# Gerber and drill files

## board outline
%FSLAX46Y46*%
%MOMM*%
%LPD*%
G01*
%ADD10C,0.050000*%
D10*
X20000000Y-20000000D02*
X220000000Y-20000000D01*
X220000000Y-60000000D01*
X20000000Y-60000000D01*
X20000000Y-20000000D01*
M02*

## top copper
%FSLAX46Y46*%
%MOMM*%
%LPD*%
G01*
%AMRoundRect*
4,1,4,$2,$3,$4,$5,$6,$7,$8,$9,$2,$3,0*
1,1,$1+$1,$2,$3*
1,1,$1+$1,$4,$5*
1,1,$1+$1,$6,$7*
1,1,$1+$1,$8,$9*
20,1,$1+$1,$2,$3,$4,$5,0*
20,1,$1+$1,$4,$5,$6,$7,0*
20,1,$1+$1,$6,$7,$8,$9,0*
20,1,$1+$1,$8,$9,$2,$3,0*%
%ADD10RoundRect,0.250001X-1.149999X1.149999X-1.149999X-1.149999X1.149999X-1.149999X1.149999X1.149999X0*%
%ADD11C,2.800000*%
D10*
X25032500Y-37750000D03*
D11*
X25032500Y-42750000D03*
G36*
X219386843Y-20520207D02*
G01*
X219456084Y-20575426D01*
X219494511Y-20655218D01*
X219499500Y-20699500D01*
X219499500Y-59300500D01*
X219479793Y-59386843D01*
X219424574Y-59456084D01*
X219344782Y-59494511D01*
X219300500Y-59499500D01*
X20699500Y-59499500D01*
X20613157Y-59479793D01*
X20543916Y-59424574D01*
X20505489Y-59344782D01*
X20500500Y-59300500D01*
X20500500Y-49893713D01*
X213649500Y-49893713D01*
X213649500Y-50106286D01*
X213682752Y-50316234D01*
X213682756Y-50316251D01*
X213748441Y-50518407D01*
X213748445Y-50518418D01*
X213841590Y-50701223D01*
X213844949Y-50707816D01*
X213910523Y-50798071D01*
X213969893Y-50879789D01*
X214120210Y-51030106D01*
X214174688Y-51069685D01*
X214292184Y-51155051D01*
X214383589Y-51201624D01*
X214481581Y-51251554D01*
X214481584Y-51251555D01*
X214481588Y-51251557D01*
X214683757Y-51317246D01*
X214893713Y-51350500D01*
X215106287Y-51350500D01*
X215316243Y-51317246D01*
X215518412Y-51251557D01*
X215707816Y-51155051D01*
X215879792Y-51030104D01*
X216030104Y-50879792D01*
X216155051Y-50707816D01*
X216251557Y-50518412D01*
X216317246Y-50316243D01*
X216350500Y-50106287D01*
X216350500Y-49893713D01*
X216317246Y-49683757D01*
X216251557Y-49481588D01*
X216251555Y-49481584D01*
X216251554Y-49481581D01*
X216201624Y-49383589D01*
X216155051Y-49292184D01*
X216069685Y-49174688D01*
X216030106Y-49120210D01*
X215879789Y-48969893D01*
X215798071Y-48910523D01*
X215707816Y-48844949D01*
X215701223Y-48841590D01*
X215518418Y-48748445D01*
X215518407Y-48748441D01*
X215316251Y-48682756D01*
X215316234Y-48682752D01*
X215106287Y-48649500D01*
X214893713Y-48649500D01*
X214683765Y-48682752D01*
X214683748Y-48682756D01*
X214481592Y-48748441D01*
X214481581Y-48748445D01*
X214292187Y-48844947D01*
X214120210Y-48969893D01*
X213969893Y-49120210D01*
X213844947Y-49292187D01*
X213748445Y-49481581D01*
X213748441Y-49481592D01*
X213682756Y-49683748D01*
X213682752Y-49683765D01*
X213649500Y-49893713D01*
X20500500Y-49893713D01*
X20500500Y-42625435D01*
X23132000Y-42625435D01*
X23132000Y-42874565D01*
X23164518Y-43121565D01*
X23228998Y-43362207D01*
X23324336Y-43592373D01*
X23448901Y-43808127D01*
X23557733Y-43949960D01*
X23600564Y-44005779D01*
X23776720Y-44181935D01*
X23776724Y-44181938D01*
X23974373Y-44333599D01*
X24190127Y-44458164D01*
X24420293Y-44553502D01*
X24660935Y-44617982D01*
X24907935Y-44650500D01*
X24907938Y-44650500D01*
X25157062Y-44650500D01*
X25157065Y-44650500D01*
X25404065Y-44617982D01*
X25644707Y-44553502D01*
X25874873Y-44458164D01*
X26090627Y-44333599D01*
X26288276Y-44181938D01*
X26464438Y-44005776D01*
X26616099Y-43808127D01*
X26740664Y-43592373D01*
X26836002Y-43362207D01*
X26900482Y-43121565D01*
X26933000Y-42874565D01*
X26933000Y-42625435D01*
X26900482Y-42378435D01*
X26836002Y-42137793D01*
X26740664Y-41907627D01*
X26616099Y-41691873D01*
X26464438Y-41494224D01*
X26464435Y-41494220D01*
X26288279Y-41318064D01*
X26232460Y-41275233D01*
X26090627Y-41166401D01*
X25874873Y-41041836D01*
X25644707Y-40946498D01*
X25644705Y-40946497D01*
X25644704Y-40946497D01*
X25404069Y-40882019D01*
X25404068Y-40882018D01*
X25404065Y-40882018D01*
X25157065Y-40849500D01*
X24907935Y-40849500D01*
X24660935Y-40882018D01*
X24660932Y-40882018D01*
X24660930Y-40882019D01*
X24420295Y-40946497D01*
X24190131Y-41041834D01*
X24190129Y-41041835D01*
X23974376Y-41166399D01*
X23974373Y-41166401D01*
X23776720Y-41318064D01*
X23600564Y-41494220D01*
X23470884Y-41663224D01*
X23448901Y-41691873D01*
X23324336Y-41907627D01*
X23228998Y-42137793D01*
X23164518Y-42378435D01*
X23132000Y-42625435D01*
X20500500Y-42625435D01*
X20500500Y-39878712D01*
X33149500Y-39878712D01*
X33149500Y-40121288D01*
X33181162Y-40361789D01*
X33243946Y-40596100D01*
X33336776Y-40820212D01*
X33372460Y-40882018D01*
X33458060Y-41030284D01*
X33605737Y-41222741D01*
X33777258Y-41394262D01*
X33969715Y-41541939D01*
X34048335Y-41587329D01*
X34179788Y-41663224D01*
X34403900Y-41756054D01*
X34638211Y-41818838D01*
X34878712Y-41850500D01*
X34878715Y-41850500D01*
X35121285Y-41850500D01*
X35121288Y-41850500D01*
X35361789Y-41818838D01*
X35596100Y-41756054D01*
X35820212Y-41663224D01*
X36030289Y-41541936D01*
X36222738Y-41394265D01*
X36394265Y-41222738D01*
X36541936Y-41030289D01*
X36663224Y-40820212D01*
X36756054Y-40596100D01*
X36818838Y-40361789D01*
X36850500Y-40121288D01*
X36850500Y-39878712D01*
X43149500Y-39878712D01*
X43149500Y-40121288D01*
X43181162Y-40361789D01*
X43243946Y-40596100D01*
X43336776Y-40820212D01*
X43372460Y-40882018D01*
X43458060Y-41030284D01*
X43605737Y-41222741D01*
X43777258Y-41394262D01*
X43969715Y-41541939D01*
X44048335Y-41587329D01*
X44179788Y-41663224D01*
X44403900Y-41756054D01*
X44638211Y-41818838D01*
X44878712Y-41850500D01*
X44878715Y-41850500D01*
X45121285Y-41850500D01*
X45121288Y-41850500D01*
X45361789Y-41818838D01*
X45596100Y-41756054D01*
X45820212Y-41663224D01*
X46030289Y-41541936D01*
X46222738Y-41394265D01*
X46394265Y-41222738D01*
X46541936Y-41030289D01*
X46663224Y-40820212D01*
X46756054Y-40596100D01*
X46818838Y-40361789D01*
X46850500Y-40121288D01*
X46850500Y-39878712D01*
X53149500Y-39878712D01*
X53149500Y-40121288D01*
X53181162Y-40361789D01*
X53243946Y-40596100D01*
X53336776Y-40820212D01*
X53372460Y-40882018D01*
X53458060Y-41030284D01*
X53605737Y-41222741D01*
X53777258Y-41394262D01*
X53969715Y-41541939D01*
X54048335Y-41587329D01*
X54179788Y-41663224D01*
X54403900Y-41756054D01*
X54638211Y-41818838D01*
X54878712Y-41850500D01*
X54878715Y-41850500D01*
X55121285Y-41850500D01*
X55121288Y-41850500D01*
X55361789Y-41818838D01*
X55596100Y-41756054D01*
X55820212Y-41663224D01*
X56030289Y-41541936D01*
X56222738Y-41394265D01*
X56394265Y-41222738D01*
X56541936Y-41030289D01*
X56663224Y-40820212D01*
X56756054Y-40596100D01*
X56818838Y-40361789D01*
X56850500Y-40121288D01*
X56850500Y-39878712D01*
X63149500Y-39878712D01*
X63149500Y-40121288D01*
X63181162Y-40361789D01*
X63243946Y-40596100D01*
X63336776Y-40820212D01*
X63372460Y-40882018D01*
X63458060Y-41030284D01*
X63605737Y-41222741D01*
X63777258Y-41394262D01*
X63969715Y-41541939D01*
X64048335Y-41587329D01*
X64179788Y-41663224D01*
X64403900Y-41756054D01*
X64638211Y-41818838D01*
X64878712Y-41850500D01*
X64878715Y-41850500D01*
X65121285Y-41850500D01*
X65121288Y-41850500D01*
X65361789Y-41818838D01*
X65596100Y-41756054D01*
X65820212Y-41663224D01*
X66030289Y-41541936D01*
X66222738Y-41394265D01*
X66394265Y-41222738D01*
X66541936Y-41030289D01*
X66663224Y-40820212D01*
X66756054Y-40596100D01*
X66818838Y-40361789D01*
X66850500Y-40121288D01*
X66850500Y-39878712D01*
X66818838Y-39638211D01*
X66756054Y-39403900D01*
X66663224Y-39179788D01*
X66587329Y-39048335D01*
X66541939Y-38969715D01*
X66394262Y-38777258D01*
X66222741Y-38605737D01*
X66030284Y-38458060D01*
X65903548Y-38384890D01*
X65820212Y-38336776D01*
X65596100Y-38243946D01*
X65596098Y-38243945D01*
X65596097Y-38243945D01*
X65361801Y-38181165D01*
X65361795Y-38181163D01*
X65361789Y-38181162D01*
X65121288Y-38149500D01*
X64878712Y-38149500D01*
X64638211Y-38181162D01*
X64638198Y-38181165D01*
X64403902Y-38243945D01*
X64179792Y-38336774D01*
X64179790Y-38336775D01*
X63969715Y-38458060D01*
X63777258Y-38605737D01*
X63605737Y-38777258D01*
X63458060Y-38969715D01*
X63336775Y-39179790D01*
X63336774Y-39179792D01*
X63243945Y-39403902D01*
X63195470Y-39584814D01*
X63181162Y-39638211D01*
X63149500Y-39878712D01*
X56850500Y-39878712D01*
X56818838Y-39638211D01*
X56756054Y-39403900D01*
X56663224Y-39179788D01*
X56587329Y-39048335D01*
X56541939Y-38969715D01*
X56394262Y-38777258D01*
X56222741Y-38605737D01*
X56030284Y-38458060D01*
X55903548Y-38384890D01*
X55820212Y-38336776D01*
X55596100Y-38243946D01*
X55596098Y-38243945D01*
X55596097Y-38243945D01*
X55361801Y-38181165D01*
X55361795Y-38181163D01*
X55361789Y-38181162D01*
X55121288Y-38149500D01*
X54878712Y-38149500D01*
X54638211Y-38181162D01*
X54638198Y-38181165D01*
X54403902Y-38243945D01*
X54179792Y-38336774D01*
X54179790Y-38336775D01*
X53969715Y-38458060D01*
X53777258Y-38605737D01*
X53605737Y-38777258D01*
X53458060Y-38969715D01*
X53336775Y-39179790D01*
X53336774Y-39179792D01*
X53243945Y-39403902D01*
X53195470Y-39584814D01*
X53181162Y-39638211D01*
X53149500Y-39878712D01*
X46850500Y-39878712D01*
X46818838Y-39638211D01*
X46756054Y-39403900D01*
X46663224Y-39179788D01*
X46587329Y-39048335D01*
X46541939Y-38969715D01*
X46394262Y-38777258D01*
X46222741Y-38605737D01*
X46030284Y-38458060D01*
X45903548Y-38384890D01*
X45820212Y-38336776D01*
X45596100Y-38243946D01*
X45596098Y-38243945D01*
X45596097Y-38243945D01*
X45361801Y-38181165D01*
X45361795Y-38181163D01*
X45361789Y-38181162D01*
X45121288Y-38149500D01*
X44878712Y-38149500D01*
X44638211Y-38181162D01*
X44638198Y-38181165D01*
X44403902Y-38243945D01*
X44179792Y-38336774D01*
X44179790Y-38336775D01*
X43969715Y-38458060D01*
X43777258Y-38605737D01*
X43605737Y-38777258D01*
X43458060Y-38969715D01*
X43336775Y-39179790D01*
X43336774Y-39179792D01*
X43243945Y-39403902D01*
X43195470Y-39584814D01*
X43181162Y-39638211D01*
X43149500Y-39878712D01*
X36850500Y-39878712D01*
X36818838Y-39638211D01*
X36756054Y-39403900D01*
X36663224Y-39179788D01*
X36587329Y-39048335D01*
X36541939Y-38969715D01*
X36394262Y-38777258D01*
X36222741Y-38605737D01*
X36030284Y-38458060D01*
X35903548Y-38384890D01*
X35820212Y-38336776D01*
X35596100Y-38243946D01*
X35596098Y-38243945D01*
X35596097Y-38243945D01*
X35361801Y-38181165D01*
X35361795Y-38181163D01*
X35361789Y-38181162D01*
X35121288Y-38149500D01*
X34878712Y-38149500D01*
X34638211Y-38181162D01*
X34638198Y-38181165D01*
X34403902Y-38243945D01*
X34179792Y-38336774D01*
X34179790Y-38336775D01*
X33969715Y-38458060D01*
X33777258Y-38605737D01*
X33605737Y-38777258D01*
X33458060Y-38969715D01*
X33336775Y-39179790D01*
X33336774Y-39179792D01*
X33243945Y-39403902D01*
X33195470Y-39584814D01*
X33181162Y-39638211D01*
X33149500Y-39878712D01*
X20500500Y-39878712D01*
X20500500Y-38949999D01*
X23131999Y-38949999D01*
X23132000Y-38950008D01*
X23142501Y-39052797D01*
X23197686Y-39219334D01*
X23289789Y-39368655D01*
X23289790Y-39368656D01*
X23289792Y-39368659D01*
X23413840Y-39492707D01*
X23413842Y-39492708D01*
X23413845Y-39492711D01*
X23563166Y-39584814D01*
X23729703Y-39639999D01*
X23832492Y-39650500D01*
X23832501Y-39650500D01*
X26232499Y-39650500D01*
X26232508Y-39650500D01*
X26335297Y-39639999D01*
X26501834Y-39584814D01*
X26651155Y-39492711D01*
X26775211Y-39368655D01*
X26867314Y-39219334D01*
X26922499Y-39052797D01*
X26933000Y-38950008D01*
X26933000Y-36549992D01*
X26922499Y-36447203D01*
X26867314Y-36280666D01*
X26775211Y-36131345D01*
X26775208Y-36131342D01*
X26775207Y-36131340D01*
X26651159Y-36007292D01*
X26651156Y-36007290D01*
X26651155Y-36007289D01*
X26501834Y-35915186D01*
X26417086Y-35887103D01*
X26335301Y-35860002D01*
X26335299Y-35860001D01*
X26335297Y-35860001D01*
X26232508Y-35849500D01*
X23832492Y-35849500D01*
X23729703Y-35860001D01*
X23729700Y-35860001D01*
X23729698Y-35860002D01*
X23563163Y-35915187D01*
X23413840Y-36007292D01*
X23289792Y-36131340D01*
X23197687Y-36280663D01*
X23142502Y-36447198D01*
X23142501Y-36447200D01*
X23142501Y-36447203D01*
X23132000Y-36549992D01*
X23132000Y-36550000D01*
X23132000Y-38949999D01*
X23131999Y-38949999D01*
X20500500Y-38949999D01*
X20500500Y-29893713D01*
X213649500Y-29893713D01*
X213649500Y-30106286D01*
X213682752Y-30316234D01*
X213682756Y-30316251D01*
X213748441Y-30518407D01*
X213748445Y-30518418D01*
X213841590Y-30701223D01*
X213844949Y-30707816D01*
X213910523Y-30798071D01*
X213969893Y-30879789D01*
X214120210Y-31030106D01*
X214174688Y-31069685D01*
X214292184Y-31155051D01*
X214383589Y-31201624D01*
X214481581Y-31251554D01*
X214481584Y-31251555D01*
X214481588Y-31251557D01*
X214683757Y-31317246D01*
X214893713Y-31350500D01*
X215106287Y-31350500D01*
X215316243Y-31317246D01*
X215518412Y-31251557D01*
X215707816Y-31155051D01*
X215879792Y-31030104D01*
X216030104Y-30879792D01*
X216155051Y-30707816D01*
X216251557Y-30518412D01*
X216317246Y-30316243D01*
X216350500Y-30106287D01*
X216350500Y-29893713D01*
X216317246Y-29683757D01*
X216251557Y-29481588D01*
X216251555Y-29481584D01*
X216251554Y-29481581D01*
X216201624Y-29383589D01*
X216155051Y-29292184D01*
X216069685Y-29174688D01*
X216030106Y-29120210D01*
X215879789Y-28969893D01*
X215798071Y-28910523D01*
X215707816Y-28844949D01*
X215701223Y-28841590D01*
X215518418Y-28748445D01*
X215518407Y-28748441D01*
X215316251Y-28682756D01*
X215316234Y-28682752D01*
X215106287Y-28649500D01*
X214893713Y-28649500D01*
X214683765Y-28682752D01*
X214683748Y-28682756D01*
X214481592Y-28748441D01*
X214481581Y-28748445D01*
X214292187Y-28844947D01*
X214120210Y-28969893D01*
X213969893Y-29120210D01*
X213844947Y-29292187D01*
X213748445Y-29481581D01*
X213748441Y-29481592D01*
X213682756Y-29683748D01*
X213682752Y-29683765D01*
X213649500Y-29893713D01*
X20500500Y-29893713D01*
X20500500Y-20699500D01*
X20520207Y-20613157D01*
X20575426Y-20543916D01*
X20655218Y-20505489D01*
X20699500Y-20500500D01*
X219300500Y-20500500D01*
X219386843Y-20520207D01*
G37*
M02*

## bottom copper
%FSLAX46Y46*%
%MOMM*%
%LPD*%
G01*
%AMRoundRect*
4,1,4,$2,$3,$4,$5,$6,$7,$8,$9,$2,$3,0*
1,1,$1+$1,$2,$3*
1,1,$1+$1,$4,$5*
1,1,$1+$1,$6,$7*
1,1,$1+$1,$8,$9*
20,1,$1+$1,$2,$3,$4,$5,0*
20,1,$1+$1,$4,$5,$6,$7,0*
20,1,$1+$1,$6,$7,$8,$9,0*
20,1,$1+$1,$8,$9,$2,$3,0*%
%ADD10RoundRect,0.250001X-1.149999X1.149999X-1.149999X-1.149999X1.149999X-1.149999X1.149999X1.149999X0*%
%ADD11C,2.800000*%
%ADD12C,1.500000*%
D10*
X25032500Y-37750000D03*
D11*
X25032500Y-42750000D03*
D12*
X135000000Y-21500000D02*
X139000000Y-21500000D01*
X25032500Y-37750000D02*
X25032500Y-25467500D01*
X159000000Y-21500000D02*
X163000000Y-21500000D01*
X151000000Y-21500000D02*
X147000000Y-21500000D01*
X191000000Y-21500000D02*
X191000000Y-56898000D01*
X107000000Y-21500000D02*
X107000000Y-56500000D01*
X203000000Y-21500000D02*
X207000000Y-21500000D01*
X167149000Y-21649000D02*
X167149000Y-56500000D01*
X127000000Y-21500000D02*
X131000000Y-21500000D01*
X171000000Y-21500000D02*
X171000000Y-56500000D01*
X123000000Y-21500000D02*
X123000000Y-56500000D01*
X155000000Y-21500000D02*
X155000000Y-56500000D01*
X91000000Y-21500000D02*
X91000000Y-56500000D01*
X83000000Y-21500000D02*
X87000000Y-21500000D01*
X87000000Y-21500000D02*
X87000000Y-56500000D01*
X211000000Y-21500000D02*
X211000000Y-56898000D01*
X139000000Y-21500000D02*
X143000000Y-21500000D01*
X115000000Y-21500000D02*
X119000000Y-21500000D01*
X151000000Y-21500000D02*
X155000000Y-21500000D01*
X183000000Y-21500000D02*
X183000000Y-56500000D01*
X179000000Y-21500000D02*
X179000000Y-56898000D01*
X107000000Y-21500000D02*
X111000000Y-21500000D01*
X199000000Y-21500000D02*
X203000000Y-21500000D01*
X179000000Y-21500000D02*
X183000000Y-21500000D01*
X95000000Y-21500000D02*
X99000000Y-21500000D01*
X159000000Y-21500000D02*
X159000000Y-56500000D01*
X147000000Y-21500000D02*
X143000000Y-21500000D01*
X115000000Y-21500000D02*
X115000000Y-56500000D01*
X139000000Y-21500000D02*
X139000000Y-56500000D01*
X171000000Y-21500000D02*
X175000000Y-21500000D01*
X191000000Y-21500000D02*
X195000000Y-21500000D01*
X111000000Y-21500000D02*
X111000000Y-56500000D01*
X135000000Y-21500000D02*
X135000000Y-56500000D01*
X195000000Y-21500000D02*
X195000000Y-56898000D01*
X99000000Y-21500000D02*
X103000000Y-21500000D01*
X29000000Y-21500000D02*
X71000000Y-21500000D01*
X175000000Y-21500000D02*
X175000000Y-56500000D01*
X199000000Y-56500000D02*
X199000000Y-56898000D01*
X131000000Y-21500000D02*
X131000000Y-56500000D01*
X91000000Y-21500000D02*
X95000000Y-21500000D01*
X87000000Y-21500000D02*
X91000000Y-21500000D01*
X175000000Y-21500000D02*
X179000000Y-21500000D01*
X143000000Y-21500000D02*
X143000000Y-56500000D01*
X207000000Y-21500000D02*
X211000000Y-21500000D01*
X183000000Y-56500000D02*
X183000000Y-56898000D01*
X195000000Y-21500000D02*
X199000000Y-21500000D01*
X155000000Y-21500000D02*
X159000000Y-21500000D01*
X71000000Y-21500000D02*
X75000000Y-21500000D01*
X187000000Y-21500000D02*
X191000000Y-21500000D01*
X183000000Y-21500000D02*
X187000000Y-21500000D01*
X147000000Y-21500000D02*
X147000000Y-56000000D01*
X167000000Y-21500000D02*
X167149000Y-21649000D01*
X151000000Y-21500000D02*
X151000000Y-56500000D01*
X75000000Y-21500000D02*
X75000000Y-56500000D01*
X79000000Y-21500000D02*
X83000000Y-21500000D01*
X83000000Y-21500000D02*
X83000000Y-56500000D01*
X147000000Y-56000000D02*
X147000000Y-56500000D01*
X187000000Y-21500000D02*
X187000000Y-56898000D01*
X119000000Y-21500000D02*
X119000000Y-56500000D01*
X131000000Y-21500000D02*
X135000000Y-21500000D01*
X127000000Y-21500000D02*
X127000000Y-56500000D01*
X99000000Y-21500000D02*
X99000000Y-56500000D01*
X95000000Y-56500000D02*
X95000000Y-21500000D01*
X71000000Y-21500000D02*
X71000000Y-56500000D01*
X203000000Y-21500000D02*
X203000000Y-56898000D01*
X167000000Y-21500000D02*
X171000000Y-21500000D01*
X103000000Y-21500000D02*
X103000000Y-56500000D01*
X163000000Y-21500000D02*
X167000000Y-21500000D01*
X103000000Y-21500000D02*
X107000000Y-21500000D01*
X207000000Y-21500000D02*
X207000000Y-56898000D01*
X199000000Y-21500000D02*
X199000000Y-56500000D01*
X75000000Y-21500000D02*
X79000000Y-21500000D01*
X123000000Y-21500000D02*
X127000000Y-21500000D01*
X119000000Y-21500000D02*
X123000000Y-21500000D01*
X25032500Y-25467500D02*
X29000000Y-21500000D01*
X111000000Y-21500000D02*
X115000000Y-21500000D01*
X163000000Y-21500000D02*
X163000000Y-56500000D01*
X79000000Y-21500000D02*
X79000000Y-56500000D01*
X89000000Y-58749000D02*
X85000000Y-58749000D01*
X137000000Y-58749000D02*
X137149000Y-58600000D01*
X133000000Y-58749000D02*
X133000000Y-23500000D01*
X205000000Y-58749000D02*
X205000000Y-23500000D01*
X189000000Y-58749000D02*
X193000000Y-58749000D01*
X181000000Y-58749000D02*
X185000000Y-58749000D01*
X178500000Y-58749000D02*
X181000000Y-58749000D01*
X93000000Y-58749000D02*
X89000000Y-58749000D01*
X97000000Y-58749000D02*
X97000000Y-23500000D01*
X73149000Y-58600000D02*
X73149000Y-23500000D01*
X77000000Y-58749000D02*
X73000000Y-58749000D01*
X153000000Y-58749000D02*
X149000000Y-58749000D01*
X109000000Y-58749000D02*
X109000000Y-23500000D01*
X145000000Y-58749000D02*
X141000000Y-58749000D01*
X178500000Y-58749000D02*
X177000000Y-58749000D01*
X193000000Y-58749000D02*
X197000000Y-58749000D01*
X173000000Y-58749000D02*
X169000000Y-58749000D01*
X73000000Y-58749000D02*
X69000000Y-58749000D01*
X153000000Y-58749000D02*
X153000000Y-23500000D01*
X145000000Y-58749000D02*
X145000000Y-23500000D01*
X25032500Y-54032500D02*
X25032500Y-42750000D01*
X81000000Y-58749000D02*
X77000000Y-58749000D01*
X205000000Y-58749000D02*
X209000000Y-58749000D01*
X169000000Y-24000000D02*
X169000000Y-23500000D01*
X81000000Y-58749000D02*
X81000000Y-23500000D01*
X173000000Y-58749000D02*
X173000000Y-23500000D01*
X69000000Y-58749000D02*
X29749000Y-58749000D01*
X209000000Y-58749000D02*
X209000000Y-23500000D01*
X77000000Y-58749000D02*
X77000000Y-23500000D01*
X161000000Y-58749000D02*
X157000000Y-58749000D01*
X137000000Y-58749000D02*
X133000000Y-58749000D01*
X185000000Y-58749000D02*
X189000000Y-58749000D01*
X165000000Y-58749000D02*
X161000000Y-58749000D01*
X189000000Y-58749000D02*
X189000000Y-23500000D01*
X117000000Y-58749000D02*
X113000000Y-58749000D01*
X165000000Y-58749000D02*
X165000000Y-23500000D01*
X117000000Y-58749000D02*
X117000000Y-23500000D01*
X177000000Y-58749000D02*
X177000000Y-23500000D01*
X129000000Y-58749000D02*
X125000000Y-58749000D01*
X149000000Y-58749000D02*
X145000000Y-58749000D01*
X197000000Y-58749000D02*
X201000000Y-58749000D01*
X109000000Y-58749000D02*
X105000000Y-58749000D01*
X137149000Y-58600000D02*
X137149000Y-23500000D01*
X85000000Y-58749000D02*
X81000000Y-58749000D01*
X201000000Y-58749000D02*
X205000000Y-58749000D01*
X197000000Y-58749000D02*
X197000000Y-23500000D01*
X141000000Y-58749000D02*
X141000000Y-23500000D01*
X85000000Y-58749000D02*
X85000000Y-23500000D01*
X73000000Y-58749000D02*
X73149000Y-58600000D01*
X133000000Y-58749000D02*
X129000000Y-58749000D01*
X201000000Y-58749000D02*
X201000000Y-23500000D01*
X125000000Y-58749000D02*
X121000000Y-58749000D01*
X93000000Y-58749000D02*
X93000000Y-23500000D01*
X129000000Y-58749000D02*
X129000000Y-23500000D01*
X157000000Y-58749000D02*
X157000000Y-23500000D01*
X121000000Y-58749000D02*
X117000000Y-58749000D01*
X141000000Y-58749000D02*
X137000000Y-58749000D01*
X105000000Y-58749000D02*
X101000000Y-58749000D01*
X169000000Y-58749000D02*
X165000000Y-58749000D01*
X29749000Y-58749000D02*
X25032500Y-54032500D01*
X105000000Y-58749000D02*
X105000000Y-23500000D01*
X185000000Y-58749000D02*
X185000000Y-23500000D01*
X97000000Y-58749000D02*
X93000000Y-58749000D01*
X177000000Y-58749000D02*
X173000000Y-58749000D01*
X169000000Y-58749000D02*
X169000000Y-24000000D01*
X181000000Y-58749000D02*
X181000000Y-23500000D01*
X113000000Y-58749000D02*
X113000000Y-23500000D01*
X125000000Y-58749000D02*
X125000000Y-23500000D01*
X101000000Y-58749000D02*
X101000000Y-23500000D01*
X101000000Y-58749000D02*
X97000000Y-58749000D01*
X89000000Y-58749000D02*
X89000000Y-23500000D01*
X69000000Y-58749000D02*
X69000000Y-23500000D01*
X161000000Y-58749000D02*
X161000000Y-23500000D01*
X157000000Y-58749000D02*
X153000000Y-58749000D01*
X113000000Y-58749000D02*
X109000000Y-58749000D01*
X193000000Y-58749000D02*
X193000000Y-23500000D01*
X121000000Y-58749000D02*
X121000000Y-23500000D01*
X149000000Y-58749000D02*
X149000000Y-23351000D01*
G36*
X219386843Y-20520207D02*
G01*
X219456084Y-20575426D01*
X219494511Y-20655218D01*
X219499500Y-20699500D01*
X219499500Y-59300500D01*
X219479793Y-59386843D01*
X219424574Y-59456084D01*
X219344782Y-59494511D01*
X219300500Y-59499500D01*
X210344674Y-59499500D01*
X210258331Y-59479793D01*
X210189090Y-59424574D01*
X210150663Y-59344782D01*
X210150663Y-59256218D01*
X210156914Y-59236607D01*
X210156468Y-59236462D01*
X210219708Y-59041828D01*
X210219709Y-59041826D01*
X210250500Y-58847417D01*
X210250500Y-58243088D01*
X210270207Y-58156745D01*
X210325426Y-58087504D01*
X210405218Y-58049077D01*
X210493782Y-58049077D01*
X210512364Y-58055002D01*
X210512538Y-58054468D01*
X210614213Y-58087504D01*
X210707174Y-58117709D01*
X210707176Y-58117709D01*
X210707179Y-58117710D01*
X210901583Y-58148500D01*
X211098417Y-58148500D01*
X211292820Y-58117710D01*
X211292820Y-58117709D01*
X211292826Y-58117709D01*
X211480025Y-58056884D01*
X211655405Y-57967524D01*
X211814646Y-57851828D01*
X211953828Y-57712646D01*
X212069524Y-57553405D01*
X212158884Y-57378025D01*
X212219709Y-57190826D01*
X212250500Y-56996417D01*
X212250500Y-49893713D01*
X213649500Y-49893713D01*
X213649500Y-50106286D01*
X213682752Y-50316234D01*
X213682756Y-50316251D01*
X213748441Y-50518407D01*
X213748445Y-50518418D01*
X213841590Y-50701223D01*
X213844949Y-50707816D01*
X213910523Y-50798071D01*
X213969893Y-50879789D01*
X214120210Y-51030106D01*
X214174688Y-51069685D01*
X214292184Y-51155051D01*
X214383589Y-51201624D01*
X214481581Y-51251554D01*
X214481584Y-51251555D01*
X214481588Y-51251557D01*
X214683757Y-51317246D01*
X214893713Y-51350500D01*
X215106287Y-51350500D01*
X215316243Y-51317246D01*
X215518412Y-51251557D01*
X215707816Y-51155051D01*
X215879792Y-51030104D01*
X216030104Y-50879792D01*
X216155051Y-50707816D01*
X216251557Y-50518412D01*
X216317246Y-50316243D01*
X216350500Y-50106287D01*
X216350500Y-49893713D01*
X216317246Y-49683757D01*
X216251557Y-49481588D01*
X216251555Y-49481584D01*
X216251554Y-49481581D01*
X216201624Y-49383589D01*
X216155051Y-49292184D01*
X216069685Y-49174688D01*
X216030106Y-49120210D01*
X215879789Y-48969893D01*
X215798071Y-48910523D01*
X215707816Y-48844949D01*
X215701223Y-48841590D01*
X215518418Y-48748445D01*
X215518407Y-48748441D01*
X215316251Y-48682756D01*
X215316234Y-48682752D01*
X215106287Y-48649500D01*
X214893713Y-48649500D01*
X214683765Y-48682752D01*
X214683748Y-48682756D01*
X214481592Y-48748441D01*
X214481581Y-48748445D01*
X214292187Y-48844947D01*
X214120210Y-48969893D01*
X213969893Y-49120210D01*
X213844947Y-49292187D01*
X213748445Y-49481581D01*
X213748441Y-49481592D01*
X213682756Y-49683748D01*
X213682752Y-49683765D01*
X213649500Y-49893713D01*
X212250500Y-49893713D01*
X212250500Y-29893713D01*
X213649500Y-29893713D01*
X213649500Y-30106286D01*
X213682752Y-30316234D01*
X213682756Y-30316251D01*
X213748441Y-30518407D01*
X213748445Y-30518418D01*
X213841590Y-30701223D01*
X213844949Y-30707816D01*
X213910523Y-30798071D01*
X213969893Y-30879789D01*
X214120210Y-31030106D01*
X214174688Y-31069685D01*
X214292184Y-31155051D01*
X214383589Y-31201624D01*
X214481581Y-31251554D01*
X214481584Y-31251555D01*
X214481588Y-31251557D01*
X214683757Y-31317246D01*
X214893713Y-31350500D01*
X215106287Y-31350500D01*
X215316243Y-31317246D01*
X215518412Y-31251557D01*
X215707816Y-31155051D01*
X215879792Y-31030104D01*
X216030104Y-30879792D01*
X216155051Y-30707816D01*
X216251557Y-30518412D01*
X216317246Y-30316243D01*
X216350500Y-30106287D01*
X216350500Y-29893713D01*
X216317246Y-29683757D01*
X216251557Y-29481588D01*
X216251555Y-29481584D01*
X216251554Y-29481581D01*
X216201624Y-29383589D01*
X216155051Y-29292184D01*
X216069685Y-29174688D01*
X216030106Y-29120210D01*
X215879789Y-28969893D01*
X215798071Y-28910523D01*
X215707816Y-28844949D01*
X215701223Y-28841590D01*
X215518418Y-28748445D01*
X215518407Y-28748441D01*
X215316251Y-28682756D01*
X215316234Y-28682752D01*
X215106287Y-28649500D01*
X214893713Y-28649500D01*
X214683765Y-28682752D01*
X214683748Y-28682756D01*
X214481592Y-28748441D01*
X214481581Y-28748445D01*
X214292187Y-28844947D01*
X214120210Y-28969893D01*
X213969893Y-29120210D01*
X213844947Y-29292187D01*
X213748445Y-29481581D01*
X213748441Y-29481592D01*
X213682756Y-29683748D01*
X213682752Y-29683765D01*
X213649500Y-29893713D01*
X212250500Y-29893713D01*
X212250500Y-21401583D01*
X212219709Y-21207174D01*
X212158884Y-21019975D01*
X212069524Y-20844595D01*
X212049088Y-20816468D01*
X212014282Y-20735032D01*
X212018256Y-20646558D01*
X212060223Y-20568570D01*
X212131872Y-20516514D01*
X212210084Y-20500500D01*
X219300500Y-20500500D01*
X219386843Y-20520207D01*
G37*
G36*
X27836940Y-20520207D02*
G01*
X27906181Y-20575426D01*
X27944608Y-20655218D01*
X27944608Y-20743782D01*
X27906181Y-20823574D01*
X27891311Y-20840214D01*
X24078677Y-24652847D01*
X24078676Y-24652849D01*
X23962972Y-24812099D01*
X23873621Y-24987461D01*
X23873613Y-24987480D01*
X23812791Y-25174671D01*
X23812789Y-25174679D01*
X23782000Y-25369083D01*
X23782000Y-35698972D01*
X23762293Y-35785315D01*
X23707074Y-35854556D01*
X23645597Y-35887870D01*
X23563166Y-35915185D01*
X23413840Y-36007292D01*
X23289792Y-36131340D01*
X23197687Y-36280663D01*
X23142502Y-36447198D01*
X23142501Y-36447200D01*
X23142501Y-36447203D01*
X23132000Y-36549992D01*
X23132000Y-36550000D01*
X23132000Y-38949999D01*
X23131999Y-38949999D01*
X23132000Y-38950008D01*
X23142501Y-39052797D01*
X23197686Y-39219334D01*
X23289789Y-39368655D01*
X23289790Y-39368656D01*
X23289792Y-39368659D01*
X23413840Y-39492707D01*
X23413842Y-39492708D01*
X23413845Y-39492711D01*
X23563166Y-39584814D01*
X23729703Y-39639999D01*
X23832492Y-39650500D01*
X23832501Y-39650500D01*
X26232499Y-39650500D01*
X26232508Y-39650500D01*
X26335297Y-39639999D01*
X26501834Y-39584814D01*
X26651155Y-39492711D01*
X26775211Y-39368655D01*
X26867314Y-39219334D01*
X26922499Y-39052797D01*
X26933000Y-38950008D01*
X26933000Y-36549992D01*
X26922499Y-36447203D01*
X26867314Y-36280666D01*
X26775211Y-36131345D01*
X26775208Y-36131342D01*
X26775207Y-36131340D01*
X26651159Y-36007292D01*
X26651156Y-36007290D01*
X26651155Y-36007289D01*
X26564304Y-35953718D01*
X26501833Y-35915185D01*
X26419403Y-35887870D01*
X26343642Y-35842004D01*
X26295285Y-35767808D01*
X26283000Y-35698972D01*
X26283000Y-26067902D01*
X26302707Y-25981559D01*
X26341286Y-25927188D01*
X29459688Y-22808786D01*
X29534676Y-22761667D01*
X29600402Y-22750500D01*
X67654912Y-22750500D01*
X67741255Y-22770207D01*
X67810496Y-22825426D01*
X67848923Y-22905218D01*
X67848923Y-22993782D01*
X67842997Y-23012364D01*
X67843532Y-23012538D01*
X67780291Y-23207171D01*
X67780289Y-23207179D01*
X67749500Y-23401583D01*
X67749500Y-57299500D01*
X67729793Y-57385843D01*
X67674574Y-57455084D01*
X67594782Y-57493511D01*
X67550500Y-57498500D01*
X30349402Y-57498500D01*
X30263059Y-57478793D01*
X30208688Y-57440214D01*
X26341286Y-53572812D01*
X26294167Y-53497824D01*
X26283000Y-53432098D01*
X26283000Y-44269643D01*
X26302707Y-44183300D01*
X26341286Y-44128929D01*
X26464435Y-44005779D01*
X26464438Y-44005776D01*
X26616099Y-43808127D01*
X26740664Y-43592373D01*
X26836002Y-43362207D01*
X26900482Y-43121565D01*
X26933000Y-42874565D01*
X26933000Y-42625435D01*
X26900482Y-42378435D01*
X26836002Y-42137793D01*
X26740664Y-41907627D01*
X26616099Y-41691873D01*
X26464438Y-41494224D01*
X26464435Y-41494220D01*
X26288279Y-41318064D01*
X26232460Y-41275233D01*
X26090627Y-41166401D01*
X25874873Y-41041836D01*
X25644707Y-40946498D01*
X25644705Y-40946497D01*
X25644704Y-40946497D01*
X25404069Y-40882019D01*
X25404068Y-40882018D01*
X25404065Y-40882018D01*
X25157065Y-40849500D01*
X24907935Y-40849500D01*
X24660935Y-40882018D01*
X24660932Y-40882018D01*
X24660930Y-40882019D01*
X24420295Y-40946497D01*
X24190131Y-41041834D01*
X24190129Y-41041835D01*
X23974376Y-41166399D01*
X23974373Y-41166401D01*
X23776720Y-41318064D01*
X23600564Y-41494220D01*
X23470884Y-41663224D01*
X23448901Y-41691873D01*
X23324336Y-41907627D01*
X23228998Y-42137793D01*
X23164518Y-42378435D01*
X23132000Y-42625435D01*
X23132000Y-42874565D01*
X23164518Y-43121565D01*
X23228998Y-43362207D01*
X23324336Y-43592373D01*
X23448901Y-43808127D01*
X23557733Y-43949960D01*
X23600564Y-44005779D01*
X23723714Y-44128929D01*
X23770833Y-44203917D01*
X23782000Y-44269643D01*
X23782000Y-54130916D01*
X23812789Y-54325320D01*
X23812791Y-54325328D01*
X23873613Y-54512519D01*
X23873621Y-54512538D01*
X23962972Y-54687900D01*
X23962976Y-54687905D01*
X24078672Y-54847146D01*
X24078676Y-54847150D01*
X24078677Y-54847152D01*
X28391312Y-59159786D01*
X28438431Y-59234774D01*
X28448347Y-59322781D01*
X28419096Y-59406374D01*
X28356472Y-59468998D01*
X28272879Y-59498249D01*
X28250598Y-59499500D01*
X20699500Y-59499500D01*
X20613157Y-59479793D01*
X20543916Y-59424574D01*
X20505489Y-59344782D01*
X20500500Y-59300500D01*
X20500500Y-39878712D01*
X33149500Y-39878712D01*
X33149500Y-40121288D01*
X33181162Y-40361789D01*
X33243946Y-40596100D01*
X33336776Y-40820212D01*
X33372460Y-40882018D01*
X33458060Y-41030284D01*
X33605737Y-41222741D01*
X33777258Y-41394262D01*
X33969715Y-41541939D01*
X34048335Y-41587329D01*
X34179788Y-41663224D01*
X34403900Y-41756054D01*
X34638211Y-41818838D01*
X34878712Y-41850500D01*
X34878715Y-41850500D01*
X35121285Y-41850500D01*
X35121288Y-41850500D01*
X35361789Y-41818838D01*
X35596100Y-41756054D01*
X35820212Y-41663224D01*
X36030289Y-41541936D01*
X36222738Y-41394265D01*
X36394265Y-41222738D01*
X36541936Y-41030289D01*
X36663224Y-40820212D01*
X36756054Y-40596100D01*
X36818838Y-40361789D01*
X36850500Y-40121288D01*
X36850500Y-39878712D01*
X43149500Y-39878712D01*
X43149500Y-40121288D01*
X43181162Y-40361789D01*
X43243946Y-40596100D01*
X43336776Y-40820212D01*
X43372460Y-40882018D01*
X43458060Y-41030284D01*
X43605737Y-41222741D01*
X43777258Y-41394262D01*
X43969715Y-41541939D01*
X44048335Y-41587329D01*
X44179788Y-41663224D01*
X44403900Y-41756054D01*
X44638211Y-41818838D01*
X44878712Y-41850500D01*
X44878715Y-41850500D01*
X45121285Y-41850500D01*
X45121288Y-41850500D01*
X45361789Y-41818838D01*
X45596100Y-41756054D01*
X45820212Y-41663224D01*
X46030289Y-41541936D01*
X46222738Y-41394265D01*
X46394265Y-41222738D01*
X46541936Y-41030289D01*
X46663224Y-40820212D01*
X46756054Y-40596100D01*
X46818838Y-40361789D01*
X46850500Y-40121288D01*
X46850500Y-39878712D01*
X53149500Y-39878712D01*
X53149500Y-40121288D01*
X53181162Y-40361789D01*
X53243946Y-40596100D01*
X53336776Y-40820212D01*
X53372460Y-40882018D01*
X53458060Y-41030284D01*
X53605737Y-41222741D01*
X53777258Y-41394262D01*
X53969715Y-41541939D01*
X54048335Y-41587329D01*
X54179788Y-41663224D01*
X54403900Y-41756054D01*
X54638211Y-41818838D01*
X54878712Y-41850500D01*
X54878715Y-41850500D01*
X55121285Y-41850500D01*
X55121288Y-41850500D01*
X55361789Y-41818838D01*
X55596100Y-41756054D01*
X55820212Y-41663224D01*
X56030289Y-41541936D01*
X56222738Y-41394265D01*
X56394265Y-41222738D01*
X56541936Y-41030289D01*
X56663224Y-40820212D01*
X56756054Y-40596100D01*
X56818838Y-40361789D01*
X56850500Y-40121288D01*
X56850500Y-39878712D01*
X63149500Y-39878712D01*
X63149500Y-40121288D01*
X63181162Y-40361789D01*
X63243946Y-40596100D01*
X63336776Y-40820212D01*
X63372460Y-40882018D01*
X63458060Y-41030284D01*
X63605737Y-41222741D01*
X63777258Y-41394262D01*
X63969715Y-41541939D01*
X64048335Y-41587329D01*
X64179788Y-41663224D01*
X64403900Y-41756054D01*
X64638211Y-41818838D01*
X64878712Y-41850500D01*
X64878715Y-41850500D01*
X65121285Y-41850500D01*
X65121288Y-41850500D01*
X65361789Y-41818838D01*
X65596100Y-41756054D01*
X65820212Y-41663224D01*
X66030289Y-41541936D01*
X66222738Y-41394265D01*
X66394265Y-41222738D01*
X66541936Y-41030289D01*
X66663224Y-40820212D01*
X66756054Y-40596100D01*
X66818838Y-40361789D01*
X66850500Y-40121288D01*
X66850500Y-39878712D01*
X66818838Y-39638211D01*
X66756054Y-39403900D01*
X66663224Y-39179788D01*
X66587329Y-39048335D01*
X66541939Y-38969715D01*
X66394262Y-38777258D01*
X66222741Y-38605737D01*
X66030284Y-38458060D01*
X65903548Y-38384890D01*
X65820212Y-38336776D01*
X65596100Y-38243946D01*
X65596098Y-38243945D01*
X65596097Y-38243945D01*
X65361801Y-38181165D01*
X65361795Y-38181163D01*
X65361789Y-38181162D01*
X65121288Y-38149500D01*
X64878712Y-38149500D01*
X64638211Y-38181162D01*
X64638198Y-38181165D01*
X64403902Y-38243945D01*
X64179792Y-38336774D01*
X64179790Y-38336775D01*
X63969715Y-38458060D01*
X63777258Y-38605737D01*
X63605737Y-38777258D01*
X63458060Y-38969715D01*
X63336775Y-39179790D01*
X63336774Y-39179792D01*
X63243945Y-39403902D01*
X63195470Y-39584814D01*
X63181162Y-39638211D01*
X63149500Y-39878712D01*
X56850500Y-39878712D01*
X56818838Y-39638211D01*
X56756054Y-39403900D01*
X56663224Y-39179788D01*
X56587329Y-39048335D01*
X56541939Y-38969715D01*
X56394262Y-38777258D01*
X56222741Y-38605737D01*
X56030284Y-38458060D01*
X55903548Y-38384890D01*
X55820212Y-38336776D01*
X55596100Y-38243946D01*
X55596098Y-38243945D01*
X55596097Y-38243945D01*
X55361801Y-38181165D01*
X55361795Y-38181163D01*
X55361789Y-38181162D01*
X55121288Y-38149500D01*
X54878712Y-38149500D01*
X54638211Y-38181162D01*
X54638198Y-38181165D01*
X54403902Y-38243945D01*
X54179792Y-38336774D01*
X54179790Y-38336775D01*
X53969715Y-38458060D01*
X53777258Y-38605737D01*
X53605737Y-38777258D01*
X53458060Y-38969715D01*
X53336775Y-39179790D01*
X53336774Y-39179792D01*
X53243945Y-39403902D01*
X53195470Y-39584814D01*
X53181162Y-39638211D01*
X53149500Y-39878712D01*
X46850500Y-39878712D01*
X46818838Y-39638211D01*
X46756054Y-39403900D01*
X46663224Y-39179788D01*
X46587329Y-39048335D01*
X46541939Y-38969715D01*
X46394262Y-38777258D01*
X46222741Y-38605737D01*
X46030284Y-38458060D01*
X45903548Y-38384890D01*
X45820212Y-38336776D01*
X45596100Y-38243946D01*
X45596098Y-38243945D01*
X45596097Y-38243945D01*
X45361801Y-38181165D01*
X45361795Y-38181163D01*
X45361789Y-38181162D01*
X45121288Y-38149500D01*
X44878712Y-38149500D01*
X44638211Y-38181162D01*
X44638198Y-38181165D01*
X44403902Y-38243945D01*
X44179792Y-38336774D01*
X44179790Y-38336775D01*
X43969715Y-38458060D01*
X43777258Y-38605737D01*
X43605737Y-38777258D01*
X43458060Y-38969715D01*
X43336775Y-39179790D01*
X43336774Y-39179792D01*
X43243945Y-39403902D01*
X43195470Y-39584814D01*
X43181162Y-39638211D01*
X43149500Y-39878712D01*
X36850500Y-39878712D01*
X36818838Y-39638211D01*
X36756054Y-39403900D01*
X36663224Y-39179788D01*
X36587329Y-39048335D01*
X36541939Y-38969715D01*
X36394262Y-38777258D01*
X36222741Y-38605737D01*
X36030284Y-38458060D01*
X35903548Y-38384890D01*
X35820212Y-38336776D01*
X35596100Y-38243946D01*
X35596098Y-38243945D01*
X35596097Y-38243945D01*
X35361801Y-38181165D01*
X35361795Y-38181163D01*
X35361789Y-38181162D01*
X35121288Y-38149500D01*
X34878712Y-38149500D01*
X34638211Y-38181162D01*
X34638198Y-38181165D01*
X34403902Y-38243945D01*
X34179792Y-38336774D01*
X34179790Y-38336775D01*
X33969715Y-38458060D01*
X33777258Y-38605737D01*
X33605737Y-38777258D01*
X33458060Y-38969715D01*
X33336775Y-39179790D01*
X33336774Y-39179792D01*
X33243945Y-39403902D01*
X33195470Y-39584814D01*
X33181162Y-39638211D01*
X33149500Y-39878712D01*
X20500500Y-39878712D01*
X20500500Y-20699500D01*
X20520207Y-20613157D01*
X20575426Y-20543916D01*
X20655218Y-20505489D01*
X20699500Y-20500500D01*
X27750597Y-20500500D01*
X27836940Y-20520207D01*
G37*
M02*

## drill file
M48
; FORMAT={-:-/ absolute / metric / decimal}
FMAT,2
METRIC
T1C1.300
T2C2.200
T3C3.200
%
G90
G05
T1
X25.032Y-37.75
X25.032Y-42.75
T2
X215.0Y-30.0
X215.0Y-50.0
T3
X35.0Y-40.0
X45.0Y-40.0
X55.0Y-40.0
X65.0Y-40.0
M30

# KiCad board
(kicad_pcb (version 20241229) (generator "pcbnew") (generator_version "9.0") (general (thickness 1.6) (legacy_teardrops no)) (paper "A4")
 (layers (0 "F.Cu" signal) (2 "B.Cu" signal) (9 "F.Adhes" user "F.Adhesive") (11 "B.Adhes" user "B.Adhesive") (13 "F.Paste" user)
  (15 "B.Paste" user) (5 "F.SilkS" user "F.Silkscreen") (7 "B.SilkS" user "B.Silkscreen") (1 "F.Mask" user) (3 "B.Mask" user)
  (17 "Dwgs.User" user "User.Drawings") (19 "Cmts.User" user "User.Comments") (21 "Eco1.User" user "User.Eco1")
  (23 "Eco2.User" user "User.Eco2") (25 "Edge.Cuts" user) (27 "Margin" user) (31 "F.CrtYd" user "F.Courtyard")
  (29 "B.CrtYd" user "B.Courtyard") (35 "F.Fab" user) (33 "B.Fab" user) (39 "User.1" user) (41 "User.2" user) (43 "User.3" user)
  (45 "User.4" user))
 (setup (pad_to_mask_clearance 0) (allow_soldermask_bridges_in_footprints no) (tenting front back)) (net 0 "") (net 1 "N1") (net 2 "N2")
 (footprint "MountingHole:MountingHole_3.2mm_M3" (layer "F.Cu") (at 35 40)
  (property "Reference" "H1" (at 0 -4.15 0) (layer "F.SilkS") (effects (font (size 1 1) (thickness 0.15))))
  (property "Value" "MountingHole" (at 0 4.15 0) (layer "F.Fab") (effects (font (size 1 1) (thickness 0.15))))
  (pad "" np_thru_hole circle (at 0 0) (size 3.2 3.2) (drill 3.2) (layers "*.Cu" "*.Mask")))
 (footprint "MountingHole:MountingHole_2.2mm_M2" (layer "F.Cu") (at 215 30)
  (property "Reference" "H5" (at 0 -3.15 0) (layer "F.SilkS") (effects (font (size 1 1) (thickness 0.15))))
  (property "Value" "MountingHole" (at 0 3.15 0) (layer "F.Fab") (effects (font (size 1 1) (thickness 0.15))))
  (pad "" np_thru_hole circle (at 0 0) (size 2.2 2.2) (drill 2.2) (layers "*.Cu" "*.Mask")))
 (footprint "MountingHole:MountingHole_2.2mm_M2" (layer "F.Cu") (at 215 50)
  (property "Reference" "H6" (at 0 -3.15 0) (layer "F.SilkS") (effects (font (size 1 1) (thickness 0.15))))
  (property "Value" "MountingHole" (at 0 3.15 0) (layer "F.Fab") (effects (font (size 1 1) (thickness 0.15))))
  (pad "" np_thru_hole circle (at 0 0) (size 2.2 2.2) (drill 2.2) (layers "*.Cu" "*.Mask")))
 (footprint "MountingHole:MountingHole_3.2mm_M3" (layer "F.Cu") (at 65 40)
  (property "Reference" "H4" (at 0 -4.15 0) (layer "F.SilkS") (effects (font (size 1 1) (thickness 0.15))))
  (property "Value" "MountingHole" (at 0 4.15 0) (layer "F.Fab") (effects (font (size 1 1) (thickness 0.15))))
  (pad "" np_thru_hole circle (at 0 0) (size 3.2 3.2) (drill 3.2) (layers "*.Cu" "*.Mask")))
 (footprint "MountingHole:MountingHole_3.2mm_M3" (layer "F.Cu") (at 55 40)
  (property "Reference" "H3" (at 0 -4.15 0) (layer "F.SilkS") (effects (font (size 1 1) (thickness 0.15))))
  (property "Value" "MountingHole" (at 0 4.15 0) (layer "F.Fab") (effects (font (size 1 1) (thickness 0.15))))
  (pad "" np_thru_hole circle (at 0 0) (size 3.2 3.2) (drill 3.2) (layers "*.Cu" "*.Mask")))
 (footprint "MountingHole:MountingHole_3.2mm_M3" (layer "F.Cu") (at 45 40)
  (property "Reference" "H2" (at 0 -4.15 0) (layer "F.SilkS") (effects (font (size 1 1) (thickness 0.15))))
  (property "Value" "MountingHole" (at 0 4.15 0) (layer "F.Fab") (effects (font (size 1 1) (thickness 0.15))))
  (pad "" np_thru_hole circle (at 0 0) (size 3.2 3.2) (drill 3.2) (layers "*.Cu" "*.Mask")))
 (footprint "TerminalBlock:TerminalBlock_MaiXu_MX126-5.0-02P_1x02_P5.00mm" (layer "F.Cu") (at 25.0325 37.75 -90)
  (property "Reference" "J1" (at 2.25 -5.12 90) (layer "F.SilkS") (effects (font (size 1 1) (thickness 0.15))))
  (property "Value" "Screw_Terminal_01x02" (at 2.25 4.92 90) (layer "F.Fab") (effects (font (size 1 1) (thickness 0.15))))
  (pad "1" thru_hole roundrect (at 0 0 270) (size 2.8 2.8) (drill 1.3) (layers "*.Cu" "*.Mask") (remove_unused_layers no)
   (roundrect_rratio 0.089286) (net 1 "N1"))
  (pad "2" thru_hole circle (at 5 0 270) (size 2.8 2.8) (drill 1.3) (layers "*.Cu" "*.Mask") (remove_unused_layers no) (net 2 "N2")))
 (gr_rect (start 20 20) (end 220 60) (stroke (width 0.05) (type solid)) (fill no) (layer "Edge.Cuts"))
 (segment (start 135 21.5) (end 139 21.5) (width 1.5) (layer "B.Cu") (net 1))
 (segment (start 25.0325 37.75) (end 25.0325 25.4675) (width 1.5) (layer "B.Cu") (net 1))
 (segment (start 159 21.5) (end 163 21.5) (width 1.5) (layer "B.Cu") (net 1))
 (segment (start 151 21.5) (end 147 21.5) (width 1.5) (layer "B.Cu") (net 1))
 (segment (start 191 21.5) (end 191 56.898) (width 1.5) (layer "B.Cu") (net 1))
 (segment (start 107 21.5) (end 107 56.5) (width 1.5) (layer "B.Cu") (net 1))
 (segment (start 203 21.5) (end 207 21.5) (width 1.5) (layer "B.Cu") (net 1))
 (segment (start 167.149 21.649) (end 167.149 56.5) (width 1.5) (layer "B.Cu") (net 1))
 (segment (start 127 21.5) (end 131 21.5) (width 1.5) (layer "B.Cu") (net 1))
 (segment (start 171 21.5) (end 171 56.5) (width 1.5) (layer "B.Cu") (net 1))
 (segment (start 123 21.5) (end 123 56.5) (width 1.5) (layer "B.Cu") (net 1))
 (segment (start 155 21.5) (end 155 56.5) (width 1.5) (layer "B.Cu") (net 1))
 (segment (start 91 21.5) (end 91 56.5) (width 1.5) (layer "B.Cu") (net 1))
 (segment (start 83 21.5) (end 87 21.5) (width 1.5) (layer "B.Cu") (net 1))
 (segment (start 87 21.5) (end 87 56.5) (width 1.5) (layer "B.Cu") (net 1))
 (segment (start 211 21.5) (end 211 56.898) (width 1.5) (layer "B.Cu") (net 1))
 (segment (start 139 21.5) (end 143 21.5) (width 1.5) (layer "B.Cu") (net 1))
 (segment (start 115 21.5) (end 119 21.5) (width 1.5) (layer "B.Cu") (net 1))
 (segment (start 151 21.5) (end 155 21.5) (width 1.5) (layer "B.Cu") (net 1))
 (segment (start 183 21.5) (end 183 56.5) (width 1.5) (layer "B.Cu") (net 1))
 (segment (start 179 21.5) (end 179 56.898) (width 1.5) (layer "B.Cu") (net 1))
 (segment (start 107 21.5) (end 111 21.5) (width 1.5) (layer "B.Cu") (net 1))
 (segment (start 199 21.5) (end 203 21.5) (width 1.5) (layer "B.Cu") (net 1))
 (segment (start 179 21.5) (end 183 21.5) (width 1.5) (layer "B.Cu") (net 1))
 (segment (start 95 21.5) (end 99 21.5) (width 1.5) (layer "B.Cu") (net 1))
 (segment (start 159 21.5) (end 159 56.5) (width 1.5) (layer "B.Cu") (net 1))
 (segment (start 147 21.5) (end 143 21.5) (width 1.5) (layer "B.Cu") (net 1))
 (segment (start 115 21.5) (end 115 56.5) (width 1.5) (layer "B.Cu") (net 1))
 (segment (start 139 21.5) (end 139 56.5) (width 1.5) (layer "B.Cu") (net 1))
 (segment (start 171 21.5) (end 175 21.5) (width 1.5) (layer "B.Cu") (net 1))
 (segment (start 191 21.5) (end 195 21.5) (width 1.5) (layer "B.Cu") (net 1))
 (segment (start 111 21.5) (end 111 56.5) (width 1.5) (layer "B.Cu") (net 1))
 (segment (start 135 21.5) (end 135 56.5) (width 1.5) (layer "B.Cu") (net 1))
 (segment (start 195 21.5) (end 195 56.898) (width 1.5) (layer "B.Cu") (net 1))
 (segment (start 99 21.5) (end 103 21.5) (width 1.5) (layer "B.Cu") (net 1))
 (segment (start 29 21.5) (end 71 21.5) (width 1.5) (layer "B.Cu") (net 1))
 (segment (start 175 21.5) (end 175 56.5) (width 1.5) (layer "B.Cu") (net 1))
 (segment (start 199 56.5) (end 199 56.898) (width 1.5) (layer "B.Cu") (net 1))
 (segment (start 131 21.5) (end 131 56.5) (width 1.5) (layer "B.Cu") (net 1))
 (segment (start 91 21.5) (end 95 21.5) (width 1.5) (layer "B.Cu") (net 1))
 (segment (start 87 21.5) (end 91 21.5) (width 1.5) (layer "B.Cu") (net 1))
 (segment (start 175 21.5) (end 179 21.5) (width 1.5) (layer "B.Cu") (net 1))
 (segment (start 143 21.5) (end 143 56.5) (width 1.5) (layer "B.Cu") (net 1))
 (segment (start 207 21.5) (end 211 21.5) (width 1.5) (layer "B.Cu") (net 1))
 (segment (start 183 56.5) (end 183 56.898) (width 1.5) (layer "B.Cu") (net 1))
 (segment (start 195 21.5) (end 199 21.5) (width 1.5) (layer "B.Cu") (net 1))
 (segment (start 155 21.5) (end 159 21.5) (width 1.5) (layer "B.Cu") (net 1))
 (segment (start 71 21.5) (end 75 21.5) (width 1.5) (layer "B.Cu") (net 1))
 (segment (start 187 21.5) (end 191 21.5) (width 1.5) (layer "B.Cu") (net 1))
 (segment (start 183 21.5) (end 187 21.5) (width 1.5) (layer "B.Cu") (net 1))
 (segment (start 147 21.5) (end 147 56) (width 1.5) (layer "B.Cu") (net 1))
 (segment (start 167 21.5) (end 167.149 21.649) (width 1.5) (layer "B.Cu") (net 1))
 (segment (start 151 21.5) (end 151 56.5) (width 1.5) (layer "B.Cu") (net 1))
 (segment (start 75 21.5) (end 75 56.5) (width 1.5) (layer "B.Cu") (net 1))
 (segment (start 79 21.5) (end 83 21.5) (width 1.5) (layer "B.Cu") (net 1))
 (segment (start 83 21.5) (end 83 56.5) (width 1.5) (layer "B.Cu") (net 1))
 (segment (start 147 56) (end 147 56.5) (width 1.5) (layer "B.Cu") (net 1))
 (segment (start 187 21.5) (end 187 56.898) (width 1.5) (layer "B.Cu") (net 1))
 (segment (start 119 21.5) (end 119 56.5) (width 1.5) (layer "B.Cu") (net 1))
 (segment (start 131 21.5) (end 135 21.5) (width 1.5) (layer "B.Cu") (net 1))
 (segment (start 127 21.5) (end 127 56.5) (width 1.5) (layer "B.Cu") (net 1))
 (segment (start 99 21.5) (end 99 56.5) (width 1.5) (layer "B.Cu") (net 1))
 (segment (start 95 56.5) (end 95 21.5) (width 1.5) (layer "B.Cu") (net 1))
 (segment (start 71 21.5) (end 71 56.5) (width 1.5) (layer "B.Cu") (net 1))
 (segment (start 203 21.5) (end 203 56.898) (width 1.5) (layer "B.Cu") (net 1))
 (segment (start 167 21.5) (end 171 21.5) (width 1.5) (layer "B.Cu") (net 1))
 (segment (start 103 21.5) (end 103 56.5) (width 1.5) (layer "B.Cu") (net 1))
 (segment (start 163 21.5) (end 167 21.5) (width 1.5) (layer "B.Cu") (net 1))
 (segment (start 103 21.5) (end 107 21.5) (width 1.5) (layer "B.Cu") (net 1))
 (segment (start 207 21.5) (end 207 56.898) (width 1.5) (layer "B.Cu") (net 1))
 (segment (start 199 21.5) (end 199 56.5) (width 1.5) (layer "B.Cu") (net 1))
 (segment (start 75 21.5) (end 79 21.5) (width 1.5) (layer "B.Cu") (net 1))
 (segment (start 123 21.5) (end 127 21.5) (width 1.5) (layer "B.Cu") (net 1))
 (segment (start 119 21.5) (end 123 21.5) (width 1.5) (layer "B.Cu") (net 1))
 (segment (start 25.0325 25.4675) (end 29 21.5) (width 1.5) (layer "B.Cu") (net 1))
 (segment (start 111 21.5) (end 115 21.5) (width 1.5) (layer "B.Cu") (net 1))
 (segment (start 163 21.5) (end 163 56.5) (width 1.5) (layer "B.Cu") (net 1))
 (segment (start 79 21.5) (end 79 56.5) (width 1.5) (layer "B.Cu") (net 1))
 (segment (start 89 58.749) (end 85 58.749) (width 1.5) (layer "B.Cu") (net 2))
 (segment (start 137 58.749) (end 137.149 58.6) (width 1.5) (layer "B.Cu") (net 2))
 (segment (start 133 58.749) (end 133 23.5) (width 1.5) (layer "B.Cu") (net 2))
 (segment (start 205 58.749) (end 205 23.5) (width 1.5) (layer "B.Cu") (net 2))
 (segment (start 189 58.749) (end 193 58.749) (width 1.5) (layer "B.Cu") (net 2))
 (segment (start 181 58.749) (end 185 58.749) (width 1.5) (layer "B.Cu") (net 2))
 (segment (start 178.5 58.749) (end 181 58.749) (width 1.5) (layer "B.Cu") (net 2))
 (segment (start 93 58.749) (end 89 58.749) (width 1.5) (layer "B.Cu") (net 2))
 (segment (start 97 58.749) (end 97 23.5) (width 1.5) (layer "B.Cu") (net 2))
 (segment (start 73.149 58.6) (end 73.149 23.5) (width 1.5) (layer "B.Cu") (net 2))
 (segment (start 77 58.749) (end 73 58.749) (width 1.5) (layer "B.Cu") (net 2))
 (segment (start 153 58.749) (end 149 58.749) (width 1.5) (layer "B.Cu") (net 2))
 (segment (start 109 58.749) (end 109 23.5) (width 1.5) (layer "B.Cu") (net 2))
 (segment (start 145 58.749) (end 141 58.749) (width 1.5) (layer "B.Cu") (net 2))
 (segment (start 178.5 58.749) (end 177 58.749) (width 1.5) (layer "B.Cu") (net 2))
 (segment (start 193 58.749) (end 197 58.749) (width 1.5) (layer "B.Cu") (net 2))
 (segment (start 173 58.749) (end 169 58.749) (width 1.5) (layer "B.Cu") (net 2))
 (segment (start 73 58.749) (end 69 58.749) (width 1.5) (layer "B.Cu") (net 2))
 (segment (start 153 58.749) (end 153 23.5) (width 1.5) (layer "B.Cu") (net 2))
 (segment (start 145 58.749) (end 145 23.5) (width 1.5) (layer "B.Cu") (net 2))
 (segment (start 25.0325 54.0325) (end 25.0325 42.75) (width 1.5) (layer "B.Cu") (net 2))
 (segment (start 81 58.749) (end 77 58.749) (width 1.5) (layer "B.Cu") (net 2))
 (segment (start 205 58.749) (end 209 58.749) (width 1.5) (layer "B.Cu") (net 2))
 (segment (start 169 24) (end 169 23.5) (width 1.5) (layer "B.Cu") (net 2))
 (segment (start 81 58.749) (end 81 23.5) (width 1.5) (layer "B.Cu") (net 2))
 (segment (start 173 58.749) (end 173 23.5) (width 1.5) (layer "B.Cu") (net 2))
 (segment (start 69 58.749) (end 29.749 58.749) (width 1.5) (layer "B.Cu") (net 2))
 (segment (start 209 58.749) (end 209 23.5) (width 1.5) (layer "B.Cu") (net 2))
 (segment (start 77 58.749) (end 77 23.5) (width 1.5) (layer "B.Cu") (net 2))
 (segment (start 161 58.749) (end 157 58.749) (width 1.5) (layer "B.Cu") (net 2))
 (segment (start 137 58.749) (end 133 58.749) (width 1.5) (layer "B.Cu") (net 2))
 (segment (start 185 58.749) (end 189 58.749) (width 1.5) (layer "B.Cu") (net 2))
 (segment (start 165 58.749) (end 161 58.749) (width 1.5) (layer "B.Cu") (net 2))
 (segment (start 189 58.749) (end 189 23.5) (width 1.5) (layer "B.Cu") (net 2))
 (segment (start 117 58.749) (end 113 58.749) (width 1.5) (layer "B.Cu") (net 2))
 (segment (start 165 58.749) (end 165 23.5) (width 1.5) (layer "B.Cu") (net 2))
 (segment (start 117 58.749) (end 117 23.5) (width 1.5) (layer "B.Cu") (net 2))
 (segment (start 177 58.749) (end 177 23.5) (width 1.5) (layer "B.Cu") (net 2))
 (segment (start 129 58.749) (end 125 58.749) (width 1.5) (layer "B.Cu") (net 2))
 (segment (start 149 58.749) (end 145 58.749) (width 1.5) (layer "B.Cu") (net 2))
 (segment (start 197 58.749) (end 201 58.749) (width 1.5) (layer "B.Cu") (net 2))
 (segment (start 109 58.749) (end 105 58.749) (width 1.5) (layer "B.Cu") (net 2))
 (segment (start 137.149 58.6) (end 137.149 23.5) (width 1.5) (layer "B.Cu") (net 2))
 (segment (start 85 58.749) (end 81 58.749) (width 1.5) (layer "B.Cu") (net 2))
 (segment (start 201 58.749) (end 205 58.749) (width 1.5) (layer "B.Cu") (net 2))
 (segment (start 197 58.749) (end 197 23.5) (width 1.5) (layer "B.Cu") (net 2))
 (segment (start 141 58.749) (end 141 23.5) (width 1.5) (layer "B.Cu") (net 2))
 (segment (start 85 58.749) (end 85 23.5) (width 1.5) (layer "B.Cu") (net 2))
 (segment (start 73 58.749) (end 73.149 58.6) (width 1.5) (layer "B.Cu") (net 2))
 (segment (start 133 58.749) (end 129 58.749) (width 1.5) (layer "B.Cu") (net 2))
 (segment (start 201 58.749) (end 201 23.5) (width 1.5) (layer "B.Cu") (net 2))
 (segment (start 125 58.749) (end 121 58.749) (width 1.5) (layer "B.Cu") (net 2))
 (segment (start 93 58.749) (end 93 23.5) (width 1.5) (layer "B.Cu") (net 2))
 (segment (start 129 58.749) (end 129 23.5) (width 1.5) (layer "B.Cu") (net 2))
 (segment (start 157 58.749) (end 157 23.5) (width 1.5) (layer "B.Cu") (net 2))
 (segment (start 121 58.749) (end 117 58.749) (width 1.5) (layer "B.Cu") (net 2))
 (segment (start 141 58.749) (end 137 58.749) (width 1.5) (layer "B.Cu") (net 2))
 (segment (start 105 58.749) (end 101 58.749) (width 1.5) (layer "B.Cu") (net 2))
 (segment (start 169 58.749) (end 165 58.749) (width 1.5) (layer "B.Cu") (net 2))
 (segment (start 29.749 58.749) (end 25.0325 54.0325) (width 1.5) (layer "B.Cu") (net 2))
 (segment (start 105 58.749) (end 105 23.5) (width 1.5) (layer "B.Cu") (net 2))
 (segment (start 185 58.749) (end 185 23.5) (width 1.5) (layer "B.Cu") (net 2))
 (segment (start 97 58.749) (end 93 58.749) (width 1.5) (layer "B.Cu") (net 2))
 (segment (start 177 58.749) (end 173 58.749) (width 1.5) (layer "B.Cu") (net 2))
 (segment (start 169 58.749) (end 169 24) (width 1.5) (layer "B.Cu") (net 2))
 (segment (start 181 58.749) (end 181 23.5) (width 1.5) (layer "B.Cu") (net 2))
 (segment (start 113 58.749) (end 113 23.5) (width 1.5) (layer "B.Cu") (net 2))
 (segment (start 125 58.749) (end 125 23.5) (width 1.5) (layer "B.Cu") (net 2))
 (segment (start 101 58.749) (end 101 23.5) (width 1.5) (layer "B.Cu") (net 2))
 (segment (start 101 58.749) (end 97 58.749) (width 1.5) (layer "B.Cu") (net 2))
 (segment (start 89 58.749) (end 89 23.5) (width 1.5) (layer "B.Cu") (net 2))
 (segment (start 69 58.749) (end 69 23.5) (width 1.5) (layer "B.Cu") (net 2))
 (segment (start 161 58.749) (end 161 23.5) (width 1.5) (layer "B.Cu") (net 2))
 (segment (start 157 58.749) (end 153 58.749) (width 1.5) (layer "B.Cu") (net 2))
 (segment (start 113 58.749) (end 109 58.749) (width 1.5) (layer "B.Cu") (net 2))
 (segment (start 193 58.749) (end 193 23.5) (width 1.5) (layer "B.Cu") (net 2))
 (segment (start 121 58.749) (end 121 23.5) (width 1.5) (layer "B.Cu") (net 2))
 (segment (start 149 58.749) (end 149 23.351) (width 1.5) (layer "B.Cu") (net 2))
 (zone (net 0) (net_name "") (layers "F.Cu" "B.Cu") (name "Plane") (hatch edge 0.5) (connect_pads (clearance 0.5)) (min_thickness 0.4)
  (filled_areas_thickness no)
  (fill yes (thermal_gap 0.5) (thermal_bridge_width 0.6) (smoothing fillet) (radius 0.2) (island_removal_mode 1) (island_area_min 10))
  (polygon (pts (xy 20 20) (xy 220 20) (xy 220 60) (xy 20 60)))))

